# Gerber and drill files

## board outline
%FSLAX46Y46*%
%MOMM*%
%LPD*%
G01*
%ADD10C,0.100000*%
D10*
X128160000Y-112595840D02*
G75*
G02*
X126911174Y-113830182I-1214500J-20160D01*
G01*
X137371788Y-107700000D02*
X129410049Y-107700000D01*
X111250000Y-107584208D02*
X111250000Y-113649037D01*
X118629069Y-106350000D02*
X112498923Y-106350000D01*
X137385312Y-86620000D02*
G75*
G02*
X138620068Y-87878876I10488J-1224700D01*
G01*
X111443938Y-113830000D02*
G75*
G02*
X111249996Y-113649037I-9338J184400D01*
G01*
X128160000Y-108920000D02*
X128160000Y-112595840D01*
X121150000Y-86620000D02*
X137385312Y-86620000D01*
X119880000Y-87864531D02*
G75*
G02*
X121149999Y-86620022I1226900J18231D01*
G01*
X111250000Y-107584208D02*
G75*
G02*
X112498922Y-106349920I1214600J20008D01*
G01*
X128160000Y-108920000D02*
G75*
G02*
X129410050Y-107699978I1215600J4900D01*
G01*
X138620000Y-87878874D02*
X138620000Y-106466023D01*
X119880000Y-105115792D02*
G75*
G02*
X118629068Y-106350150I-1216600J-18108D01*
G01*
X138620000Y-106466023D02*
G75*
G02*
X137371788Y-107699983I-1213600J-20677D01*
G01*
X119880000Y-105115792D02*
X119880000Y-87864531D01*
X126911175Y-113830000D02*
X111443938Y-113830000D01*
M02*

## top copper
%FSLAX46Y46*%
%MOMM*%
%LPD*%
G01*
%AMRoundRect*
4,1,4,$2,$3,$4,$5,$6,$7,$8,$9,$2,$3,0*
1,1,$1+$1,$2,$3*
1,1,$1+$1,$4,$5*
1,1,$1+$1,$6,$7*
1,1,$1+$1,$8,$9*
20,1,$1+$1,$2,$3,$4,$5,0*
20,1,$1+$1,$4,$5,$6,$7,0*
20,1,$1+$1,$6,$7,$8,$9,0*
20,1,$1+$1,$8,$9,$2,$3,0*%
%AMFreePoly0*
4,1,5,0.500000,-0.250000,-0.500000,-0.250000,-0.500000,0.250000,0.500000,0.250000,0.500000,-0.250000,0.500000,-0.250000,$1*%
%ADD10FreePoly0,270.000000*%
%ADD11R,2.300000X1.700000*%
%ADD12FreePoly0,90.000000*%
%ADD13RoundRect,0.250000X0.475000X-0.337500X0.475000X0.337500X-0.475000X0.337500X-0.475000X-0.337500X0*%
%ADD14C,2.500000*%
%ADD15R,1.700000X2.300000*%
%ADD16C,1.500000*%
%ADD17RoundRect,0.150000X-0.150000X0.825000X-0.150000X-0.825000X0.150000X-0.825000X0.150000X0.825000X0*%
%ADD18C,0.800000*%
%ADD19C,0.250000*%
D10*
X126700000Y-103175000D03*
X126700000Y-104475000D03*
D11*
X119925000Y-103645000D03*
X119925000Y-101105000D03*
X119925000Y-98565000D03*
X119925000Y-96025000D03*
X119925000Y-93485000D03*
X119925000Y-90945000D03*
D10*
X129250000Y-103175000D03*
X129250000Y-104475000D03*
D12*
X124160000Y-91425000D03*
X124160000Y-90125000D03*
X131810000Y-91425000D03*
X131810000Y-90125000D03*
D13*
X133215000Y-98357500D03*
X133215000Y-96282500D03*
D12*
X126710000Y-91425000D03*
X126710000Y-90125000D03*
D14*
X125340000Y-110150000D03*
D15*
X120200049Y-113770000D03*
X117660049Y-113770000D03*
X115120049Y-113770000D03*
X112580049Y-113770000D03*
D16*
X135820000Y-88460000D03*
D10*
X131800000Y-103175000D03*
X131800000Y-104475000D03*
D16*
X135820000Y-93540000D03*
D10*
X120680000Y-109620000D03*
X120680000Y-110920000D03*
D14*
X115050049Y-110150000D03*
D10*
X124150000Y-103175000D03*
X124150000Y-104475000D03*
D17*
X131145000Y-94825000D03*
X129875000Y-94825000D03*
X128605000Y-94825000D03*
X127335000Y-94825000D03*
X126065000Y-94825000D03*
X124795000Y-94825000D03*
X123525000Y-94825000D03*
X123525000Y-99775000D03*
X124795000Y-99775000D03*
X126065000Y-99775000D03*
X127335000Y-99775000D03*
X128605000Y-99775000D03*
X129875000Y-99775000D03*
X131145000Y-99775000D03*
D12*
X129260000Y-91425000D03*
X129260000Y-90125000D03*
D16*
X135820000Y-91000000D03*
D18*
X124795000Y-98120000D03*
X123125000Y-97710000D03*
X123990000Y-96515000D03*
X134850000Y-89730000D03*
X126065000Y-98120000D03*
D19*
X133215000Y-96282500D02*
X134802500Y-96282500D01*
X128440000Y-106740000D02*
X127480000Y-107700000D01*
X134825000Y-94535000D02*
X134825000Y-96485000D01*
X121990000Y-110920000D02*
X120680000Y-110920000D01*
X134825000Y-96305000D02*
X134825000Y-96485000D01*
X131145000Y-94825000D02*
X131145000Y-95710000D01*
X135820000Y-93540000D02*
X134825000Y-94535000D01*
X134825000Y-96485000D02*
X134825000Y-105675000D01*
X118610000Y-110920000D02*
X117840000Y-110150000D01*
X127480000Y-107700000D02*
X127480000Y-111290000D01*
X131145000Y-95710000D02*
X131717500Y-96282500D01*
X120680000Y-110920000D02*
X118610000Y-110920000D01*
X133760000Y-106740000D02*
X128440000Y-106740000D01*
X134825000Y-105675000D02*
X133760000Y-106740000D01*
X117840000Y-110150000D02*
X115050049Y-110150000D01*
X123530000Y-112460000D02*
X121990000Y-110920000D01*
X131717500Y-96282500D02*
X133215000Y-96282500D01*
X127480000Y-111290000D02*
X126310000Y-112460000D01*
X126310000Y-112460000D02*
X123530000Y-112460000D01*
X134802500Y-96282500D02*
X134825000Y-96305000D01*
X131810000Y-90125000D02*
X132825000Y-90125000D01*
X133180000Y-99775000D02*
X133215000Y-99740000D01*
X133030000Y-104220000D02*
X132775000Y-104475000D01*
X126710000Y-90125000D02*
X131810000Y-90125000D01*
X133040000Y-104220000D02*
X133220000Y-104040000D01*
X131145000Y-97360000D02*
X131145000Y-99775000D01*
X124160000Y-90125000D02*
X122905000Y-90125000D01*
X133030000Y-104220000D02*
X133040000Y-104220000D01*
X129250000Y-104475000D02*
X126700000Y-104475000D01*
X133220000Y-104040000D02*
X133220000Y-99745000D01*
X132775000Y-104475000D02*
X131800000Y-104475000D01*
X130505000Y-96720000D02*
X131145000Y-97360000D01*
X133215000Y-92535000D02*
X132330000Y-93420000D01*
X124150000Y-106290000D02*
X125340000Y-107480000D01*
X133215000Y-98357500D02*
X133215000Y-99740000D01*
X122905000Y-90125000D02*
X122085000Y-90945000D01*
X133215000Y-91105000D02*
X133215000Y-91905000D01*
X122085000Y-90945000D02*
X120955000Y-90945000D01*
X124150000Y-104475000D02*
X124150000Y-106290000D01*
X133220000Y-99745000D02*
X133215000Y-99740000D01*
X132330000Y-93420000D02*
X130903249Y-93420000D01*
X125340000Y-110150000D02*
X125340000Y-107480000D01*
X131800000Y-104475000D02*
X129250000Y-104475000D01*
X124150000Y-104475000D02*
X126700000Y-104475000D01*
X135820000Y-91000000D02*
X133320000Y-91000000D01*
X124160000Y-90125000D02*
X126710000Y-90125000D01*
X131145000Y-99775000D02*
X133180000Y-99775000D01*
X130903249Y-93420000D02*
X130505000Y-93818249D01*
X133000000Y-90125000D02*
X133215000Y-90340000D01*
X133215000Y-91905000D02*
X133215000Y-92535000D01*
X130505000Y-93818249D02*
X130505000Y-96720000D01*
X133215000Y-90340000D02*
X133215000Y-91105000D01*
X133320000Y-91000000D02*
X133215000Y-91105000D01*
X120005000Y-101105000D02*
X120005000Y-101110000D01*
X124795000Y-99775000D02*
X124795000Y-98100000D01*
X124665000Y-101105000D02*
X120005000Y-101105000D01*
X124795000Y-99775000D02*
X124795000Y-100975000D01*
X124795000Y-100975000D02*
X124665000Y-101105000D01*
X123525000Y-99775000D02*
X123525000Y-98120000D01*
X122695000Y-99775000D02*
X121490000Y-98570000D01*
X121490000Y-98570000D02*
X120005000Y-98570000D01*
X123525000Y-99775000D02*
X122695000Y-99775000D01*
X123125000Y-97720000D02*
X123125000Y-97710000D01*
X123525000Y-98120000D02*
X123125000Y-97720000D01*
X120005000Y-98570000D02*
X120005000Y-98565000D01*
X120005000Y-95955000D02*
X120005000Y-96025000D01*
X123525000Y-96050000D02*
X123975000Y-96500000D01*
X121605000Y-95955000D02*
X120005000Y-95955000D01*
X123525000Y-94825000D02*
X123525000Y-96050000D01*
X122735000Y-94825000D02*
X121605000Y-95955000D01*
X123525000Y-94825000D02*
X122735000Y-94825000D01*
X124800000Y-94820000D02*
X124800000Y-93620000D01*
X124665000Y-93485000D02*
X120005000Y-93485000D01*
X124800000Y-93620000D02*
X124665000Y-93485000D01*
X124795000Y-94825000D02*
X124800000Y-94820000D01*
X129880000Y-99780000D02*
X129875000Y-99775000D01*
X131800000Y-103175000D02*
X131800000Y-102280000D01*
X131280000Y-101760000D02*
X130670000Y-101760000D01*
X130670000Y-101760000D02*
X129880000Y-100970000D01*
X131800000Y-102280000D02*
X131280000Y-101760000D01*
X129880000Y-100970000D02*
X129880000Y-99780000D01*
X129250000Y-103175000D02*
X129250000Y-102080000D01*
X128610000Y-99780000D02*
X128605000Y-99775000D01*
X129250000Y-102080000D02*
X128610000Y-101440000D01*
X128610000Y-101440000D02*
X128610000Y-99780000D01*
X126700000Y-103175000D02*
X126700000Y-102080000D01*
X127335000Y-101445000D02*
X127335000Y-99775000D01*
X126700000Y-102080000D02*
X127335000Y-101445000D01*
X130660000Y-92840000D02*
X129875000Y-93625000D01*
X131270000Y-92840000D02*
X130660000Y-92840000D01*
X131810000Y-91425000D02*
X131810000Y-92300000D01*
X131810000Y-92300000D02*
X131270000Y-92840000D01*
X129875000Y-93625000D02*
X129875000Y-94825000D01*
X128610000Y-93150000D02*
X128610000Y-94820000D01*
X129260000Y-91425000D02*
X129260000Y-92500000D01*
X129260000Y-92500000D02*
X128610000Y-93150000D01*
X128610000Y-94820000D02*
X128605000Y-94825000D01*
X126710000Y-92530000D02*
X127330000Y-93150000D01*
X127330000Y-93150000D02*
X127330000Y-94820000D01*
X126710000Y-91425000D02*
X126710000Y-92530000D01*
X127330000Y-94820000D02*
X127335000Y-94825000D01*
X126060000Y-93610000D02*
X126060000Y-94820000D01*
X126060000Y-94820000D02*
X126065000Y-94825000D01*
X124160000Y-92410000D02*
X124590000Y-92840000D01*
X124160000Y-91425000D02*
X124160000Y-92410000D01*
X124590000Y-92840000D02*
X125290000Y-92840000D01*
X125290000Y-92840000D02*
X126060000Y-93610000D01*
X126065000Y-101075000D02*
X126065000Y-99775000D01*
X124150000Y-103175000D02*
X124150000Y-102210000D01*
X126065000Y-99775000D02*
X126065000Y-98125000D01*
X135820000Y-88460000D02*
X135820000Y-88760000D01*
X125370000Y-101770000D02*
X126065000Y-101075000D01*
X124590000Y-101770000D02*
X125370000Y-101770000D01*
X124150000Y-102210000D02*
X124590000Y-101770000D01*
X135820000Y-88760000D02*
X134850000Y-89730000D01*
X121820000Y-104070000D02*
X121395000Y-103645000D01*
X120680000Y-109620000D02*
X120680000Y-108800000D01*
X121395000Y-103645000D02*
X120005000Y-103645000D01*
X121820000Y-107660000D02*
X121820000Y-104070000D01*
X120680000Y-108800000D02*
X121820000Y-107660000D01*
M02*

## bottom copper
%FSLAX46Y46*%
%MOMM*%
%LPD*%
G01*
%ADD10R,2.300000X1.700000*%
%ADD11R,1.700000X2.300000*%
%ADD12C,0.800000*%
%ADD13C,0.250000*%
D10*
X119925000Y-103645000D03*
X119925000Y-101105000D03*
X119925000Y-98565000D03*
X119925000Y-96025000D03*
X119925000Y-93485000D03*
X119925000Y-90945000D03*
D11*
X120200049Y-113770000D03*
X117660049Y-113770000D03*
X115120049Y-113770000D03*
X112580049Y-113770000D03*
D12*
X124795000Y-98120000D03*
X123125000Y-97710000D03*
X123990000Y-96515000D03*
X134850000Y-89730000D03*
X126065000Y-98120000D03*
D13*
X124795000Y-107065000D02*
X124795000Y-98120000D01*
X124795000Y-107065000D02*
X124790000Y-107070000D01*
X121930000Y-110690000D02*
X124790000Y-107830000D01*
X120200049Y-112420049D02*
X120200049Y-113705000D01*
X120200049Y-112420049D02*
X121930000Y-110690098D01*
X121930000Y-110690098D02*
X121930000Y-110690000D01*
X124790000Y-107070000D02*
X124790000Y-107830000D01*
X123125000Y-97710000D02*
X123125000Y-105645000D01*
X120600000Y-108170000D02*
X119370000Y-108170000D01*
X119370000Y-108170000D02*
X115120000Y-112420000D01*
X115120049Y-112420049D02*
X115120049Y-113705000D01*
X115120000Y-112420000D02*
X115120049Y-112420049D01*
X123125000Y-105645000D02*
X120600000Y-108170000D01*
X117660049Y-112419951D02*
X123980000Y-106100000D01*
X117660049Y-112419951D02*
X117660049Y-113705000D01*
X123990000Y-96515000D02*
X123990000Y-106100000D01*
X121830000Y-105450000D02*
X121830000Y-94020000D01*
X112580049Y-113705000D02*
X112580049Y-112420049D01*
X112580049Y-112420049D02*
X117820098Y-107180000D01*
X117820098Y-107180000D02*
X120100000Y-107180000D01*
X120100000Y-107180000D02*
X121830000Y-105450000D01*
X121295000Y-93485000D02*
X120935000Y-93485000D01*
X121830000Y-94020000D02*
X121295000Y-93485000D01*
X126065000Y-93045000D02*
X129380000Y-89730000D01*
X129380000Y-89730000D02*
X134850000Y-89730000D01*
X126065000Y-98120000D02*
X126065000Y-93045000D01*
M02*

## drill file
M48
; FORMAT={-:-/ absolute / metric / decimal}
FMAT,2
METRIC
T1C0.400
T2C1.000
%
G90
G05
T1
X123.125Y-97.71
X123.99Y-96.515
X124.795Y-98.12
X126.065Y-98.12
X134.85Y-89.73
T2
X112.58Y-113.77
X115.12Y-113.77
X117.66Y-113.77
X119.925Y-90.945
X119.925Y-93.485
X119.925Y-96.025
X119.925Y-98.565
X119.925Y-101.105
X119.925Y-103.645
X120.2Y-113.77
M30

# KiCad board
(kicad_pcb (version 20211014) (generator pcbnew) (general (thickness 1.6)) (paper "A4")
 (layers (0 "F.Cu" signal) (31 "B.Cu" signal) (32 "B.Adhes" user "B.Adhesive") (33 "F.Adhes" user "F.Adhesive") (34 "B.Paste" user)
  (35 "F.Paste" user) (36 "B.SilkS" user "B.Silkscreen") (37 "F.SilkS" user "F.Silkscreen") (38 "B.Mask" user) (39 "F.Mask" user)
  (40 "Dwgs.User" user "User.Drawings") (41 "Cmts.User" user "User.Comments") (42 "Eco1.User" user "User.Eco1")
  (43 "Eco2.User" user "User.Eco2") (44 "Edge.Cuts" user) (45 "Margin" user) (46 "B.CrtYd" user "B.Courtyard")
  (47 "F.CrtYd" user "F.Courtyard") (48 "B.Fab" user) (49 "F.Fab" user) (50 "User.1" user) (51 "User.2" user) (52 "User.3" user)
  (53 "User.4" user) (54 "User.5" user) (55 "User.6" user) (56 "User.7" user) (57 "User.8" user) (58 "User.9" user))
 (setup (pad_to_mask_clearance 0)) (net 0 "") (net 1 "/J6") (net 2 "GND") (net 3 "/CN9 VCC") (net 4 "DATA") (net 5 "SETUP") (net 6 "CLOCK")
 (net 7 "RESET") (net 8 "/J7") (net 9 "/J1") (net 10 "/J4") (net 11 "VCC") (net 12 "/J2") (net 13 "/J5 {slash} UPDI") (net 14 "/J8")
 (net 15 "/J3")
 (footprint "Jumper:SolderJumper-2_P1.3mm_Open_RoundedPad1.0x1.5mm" (layer "F.Cu") (at 126.7 103.825 -90)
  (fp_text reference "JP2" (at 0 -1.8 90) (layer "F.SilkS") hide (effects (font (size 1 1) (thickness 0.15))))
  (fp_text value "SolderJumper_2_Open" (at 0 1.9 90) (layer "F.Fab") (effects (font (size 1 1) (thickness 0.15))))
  (pad "1" smd custom (at -0.65 0 270) (size 1 0.5) (layers "F.Cu" "F.Mask") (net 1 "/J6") (zone_connect 2)
   (options (clearance outline) (anchor rect)) (primitives))
  (pad "2" smd custom (at 0.65 0 270) (size 1 0.5) (layers "F.Cu" "F.Mask") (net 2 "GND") (zone_connect 2)
   (options (clearance outline) (anchor rect)) (primitives)))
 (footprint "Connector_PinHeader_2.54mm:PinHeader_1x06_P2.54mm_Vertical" (layer "F.Cu") (at 119.925 103.645 180)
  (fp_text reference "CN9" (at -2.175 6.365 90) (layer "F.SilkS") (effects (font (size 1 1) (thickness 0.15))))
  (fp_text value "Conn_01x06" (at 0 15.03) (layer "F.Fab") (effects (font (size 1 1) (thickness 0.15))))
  (pad "1" thru_hole rect (at 0 0 180) (size 2.3 1.7) (drill 1) (layers *.Cu *.Mask) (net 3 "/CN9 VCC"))
  (pad "2" thru_hole rect (at 0 2.54 180) (size 2.3 1.7) (drill 1) (layers *.Cu *.Mask) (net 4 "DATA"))
  (pad "3" thru_hole rect (at 0 5.08 180) (size 2.3 1.7) (drill 1) (layers *.Cu *.Mask) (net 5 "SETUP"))
  (pad "4" thru_hole rect (at 0 7.62 180) (size 2.3 1.7) (drill 1) (layers *.Cu *.Mask) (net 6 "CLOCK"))
  (pad "5" thru_hole rect (at 0 10.16 180) (size 2.3 1.7) (drill 1) (layers *.Cu *.Mask) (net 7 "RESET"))
  (pad "6" thru_hole rect (at 0 12.7 180) (size 2.3 1.7) (drill 1) (layers *.Cu *.Mask) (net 2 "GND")))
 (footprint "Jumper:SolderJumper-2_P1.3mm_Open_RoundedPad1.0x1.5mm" (layer "F.Cu") (at 129.25 103.825 -90)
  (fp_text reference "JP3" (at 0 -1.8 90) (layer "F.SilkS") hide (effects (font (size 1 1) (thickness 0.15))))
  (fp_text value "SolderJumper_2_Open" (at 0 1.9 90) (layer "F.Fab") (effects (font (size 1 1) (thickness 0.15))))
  (pad "1" smd custom (at -0.65 0 270) (size 1 0.5) (layers "F.Cu" "F.Mask") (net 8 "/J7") (zone_connect 2)
   (options (clearance outline) (anchor rect)) (primitives))
  (pad "2" smd custom (at 0.65 0 270) (size 1 0.5) (layers "F.Cu" "F.Mask") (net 2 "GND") (zone_connect 2)
   (options (clearance outline) (anchor rect)) (primitives)))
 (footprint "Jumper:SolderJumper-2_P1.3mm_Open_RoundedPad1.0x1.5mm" (layer "F.Cu") (at 124.16 90.775 90)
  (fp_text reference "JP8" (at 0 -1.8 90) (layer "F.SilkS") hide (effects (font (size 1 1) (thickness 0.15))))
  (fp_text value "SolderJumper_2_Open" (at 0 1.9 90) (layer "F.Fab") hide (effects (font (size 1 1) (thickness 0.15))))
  (pad "1" smd custom (at -0.65 0 90) (size 1 0.5) (layers "F.Cu" "F.Mask") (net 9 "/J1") (zone_connect 2)
   (options (clearance outline) (anchor rect)) (primitives))
  (pad "2" smd custom (at 0.65 0 90) (size 1 0.5) (layers "F.Cu" "F.Mask") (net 2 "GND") (zone_connect 2)
   (options (clearance outline) (anchor rect)) (primitives)))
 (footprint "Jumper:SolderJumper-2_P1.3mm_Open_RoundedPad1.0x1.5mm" (layer "F.Cu") (at 131.81 90.775 90)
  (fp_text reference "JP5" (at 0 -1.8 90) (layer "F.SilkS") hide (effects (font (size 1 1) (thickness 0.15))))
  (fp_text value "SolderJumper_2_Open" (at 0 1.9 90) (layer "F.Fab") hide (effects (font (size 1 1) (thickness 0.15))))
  (pad "1" smd custom (at -0.65 0 90) (size 1 0.5) (layers "F.Cu" "F.Mask") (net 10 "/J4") (zone_connect 2)
   (options (clearance outline) (anchor rect)) (primitives))
  (pad "2" smd custom (at 0.65 0 90) (size 1 0.5) (layers "F.Cu" "F.Mask") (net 2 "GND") (zone_connect 2)
   (options (clearance outline) (anchor rect)) (primitives)))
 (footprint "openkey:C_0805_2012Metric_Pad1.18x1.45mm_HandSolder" (layer "F.Cu") (at 133.215 97.32 90)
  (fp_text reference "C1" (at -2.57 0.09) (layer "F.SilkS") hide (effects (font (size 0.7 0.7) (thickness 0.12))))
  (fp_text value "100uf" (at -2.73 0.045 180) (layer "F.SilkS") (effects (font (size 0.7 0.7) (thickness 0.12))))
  (pad "1" smd roundrect (at -1.0375 0 90) (size 1.175 1.45) (layers "F.Cu" "F.Paste" "F.Mask") (roundrect_rratio 0.2127659574)
   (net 2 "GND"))
  (pad "2" smd roundrect (at 1.0375 0 90) (size 1.175 1.45) (layers "F.Cu" "F.Paste" "F.Mask") (roundrect_rratio 0.2127659574)
   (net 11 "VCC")))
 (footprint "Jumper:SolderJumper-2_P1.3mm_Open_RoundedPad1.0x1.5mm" (layer "F.Cu") (at 126.71 90.775 90)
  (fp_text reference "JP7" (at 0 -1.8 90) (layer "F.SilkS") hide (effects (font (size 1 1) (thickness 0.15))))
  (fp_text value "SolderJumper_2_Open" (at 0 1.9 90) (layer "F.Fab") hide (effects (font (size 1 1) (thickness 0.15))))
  (pad "1" smd custom (at -0.65 0 90) (size 1 0.5) (layers "F.Cu" "F.Mask") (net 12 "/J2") (zone_connect 2)
   (options (clearance outline) (anchor rect)) (primitives))
  (pad "2" smd custom (at 0.65 0 90) (size 1 0.5) (layers "F.Cu" "F.Mask") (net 2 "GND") (zone_connect 2)
   (options (clearance outline) (anchor rect)) (primitives)))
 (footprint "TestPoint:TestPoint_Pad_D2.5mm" (layer "F.Cu") (at 125.34 110.12)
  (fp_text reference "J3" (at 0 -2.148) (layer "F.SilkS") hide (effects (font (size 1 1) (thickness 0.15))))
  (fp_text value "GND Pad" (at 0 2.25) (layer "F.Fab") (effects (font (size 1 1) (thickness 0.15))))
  (pad "1" smd circle (at 0 0.03) (size 2.5 2.5) (layers "F.Cu" "F.Mask") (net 2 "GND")))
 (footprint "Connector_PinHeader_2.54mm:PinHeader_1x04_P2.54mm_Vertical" (layer "F.Cu") (at 120.200049 113.77 -90)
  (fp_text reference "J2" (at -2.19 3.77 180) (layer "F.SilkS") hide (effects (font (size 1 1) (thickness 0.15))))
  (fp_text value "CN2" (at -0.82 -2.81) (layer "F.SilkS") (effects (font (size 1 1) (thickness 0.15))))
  (pad "1" thru_hole rect (at 0 0 270) (size 2.3 1.7) (drill 1) (layers *.Cu *.Mask) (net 4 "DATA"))
  (pad "2" thru_hole rect (at 0 2.54 270) (size 2.3 1.7) (drill 1) (layers *.Cu *.Mask) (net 6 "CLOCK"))
  (pad "3" thru_hole rect (at 0 5.08 270) (size 2.3 1.7) (drill 1) (layers *.Cu *.Mask) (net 5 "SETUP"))
  (pad "4" thru_hole rect (at 0 7.62 270) (size 2.3 1.7) (drill 1) (layers *.Cu *.Mask) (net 7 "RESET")))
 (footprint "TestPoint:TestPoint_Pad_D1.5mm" (layer "F.Cu") (at 135.82 88.46 90)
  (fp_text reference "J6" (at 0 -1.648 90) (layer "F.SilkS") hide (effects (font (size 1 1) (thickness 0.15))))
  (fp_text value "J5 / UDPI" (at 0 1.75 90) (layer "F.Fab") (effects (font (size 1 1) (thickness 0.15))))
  (pad "1" smd circle (at 0 0 90) (size 1.5 1.5) (layers "F.Cu" "F.Mask") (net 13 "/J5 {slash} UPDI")))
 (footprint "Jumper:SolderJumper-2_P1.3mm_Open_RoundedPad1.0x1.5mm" (layer "F.Cu") (at 131.8 103.825 -90)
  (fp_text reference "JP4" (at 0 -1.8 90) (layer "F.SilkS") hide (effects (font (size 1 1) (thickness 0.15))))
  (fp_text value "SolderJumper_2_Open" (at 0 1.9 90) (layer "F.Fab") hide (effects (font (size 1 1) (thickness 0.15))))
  (pad "1" smd custom (at -0.65 0 270) (size 1 0.5) (layers "F.Cu" "F.Mask") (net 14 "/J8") (zone_connect 2)
   (options (clearance outline) (anchor rect)) (primitives))
  (pad "2" smd custom (at 0.65 0 270) (size 1 0.5) (layers "F.Cu" "F.Mask") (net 2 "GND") (zone_connect 2)
   (options (clearance outline) (anchor rect)) (primitives)))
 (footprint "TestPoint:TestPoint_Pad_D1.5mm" (layer "F.Cu") (at 135.82 93.54 90)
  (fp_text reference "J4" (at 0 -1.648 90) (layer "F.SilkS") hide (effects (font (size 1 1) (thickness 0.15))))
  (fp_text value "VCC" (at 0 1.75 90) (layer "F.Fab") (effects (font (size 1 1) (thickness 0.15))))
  (pad "1" smd circle (at 0 0 90) (size 1.5 1.5) (layers "F.Cu" "F.Mask") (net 11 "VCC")))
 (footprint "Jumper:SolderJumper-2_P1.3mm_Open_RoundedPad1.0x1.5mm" (layer "F.Cu") (at 120.68 110.27 -90)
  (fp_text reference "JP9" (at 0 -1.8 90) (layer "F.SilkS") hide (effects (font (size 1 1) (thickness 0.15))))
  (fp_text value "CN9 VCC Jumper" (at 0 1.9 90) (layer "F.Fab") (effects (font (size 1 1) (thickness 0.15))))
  (pad "1" smd custom (at -0.65 0 270) (size 1 0.5) (layers "F.Cu" "F.Mask") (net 3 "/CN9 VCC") (zone_connect 2)
   (options (clearance outline) (anchor rect)) (primitives))
  (pad "2" smd custom (at 0.65 0 270) (size 1 0.5) (layers "F.Cu" "F.Mask") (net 11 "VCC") (zone_connect 2)
   (options (clearance outline) (anchor rect)) (primitives)))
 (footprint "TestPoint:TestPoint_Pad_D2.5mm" (layer "F.Cu") (at 115.050049 110.15 90)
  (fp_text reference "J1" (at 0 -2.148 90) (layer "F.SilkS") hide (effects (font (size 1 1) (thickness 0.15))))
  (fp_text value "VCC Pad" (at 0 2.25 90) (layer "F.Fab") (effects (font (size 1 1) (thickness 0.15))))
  (pad "1" smd circle (at 0 0 90) (size 2.5 2.5) (layers "F.Cu" "F.Mask") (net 11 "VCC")))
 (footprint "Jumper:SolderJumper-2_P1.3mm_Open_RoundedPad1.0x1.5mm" (layer "F.Cu") (at 124.15 103.825 -90)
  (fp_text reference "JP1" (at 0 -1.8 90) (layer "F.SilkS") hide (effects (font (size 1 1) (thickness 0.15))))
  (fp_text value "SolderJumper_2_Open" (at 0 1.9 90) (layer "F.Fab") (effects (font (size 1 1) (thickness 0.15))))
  (pad "1" smd custom (at -0.65 0 270) (size 1 0.5) (layers "F.Cu" "F.Mask") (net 13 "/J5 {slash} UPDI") (zone_connect 2)
   (options (clearance outline) (anchor rect)) (primitives))
  (pad "2" smd custom (at 0.65 0 270) (size 1 0.5) (layers "F.Cu" "F.Mask") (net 2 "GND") (zone_connect 2)
   (options (clearance outline) (anchor rect)) (primitives)))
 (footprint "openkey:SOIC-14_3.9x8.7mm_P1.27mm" (layer "F.Cu") (at 127.335 97.3 -90)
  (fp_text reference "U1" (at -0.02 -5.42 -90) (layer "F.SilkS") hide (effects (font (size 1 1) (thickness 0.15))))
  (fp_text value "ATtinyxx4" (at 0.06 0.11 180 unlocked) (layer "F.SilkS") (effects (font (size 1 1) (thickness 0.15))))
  (pad "1" smd roundrect (at -2.475 -3.81 270) (size 1.95 0.6) (layers "F.Cu" "F.Paste" "F.Mask") (roundrect_rratio 0.25) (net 11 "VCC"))
  (pad "2" smd roundrect (at -2.475 -2.54 270) (size 1.95 0.6) (layers "F.Cu" "F.Paste" "F.Mask") (roundrect_rratio 0.25) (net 10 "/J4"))
  (pad "3" smd roundrect (at -2.475 -1.27 270) (size 1.95 0.6) (layers "F.Cu" "F.Paste" "F.Mask") (roundrect_rratio 0.25) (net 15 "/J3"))
  (pad "4" smd roundrect (at -2.475 0 270) (size 1.95 0.6) (layers "F.Cu" "F.Paste" "F.Mask") (roundrect_rratio 0.25) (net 12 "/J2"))
  (pad "5" smd roundrect (at -2.475 1.27 270) (size 1.95 0.6) (layers "F.Cu" "F.Paste" "F.Mask") (roundrect_rratio 0.25) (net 9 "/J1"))
  (pad "6" smd roundrect (at -2.475 2.54 270) (size 1.95 0.6) (layers "F.Cu" "F.Paste" "F.Mask") (roundrect_rratio 0.25) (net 7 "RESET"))
  (pad "7" smd roundrect (at -2.475 3.81 270) (size 1.95 0.6) (layers "F.Cu" "F.Paste" "F.Mask") (roundrect_rratio 0.25) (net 6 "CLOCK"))
  (pad "8" smd roundrect (at 2.475 3.81 270) (size 1.95 0.6) (layers "F.Cu" "F.Paste" "F.Mask") (roundrect_rratio 0.25) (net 5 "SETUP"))
  (pad "9" smd roundrect (at 2.475 2.54 270) (size 1.95 0.6) (layers "F.Cu" "F.Paste" "F.Mask") (roundrect_rratio 0.25) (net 4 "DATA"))
  (pad "10" smd roundrect (at 2.475 1.27 270) (size 1.95 0.6) (layers "F.Cu" "F.Paste" "F.Mask") (roundrect_rratio 0.25)
   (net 13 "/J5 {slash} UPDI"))
  (pad "11" smd roundrect (at 2.475 0 270) (size 1.95 0.6) (layers "F.Cu" "F.Paste" "F.Mask") (roundrect_rratio 0.25) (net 1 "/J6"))
  (pad "12" smd roundrect (at 2.475 -1.27 270) (size 1.95 0.6) (layers "F.Cu" "F.Paste" "F.Mask") (roundrect_rratio 0.25) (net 8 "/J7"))
  (pad "13" smd roundrect (at 2.475 -2.54 270) (size 1.95 0.6) (layers "F.Cu" "F.Paste" "F.Mask") (roundrect_rratio 0.25) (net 14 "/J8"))
  (pad "14" smd roundrect (at 2.475 -3.81 270) (size 1.95 0.6) (layers "F.Cu" "F.Paste" "F.Mask") (roundrect_rratio 0.25) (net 2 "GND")))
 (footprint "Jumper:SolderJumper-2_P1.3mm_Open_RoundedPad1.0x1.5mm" (layer "F.Cu") (at 129.26 90.775 90)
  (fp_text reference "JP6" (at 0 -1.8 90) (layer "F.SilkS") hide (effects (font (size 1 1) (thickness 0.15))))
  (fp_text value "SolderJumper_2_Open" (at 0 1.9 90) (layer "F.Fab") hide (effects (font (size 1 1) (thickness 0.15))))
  (pad "1" smd custom (at -0.65 0 90) (size 1 0.5) (layers "F.Cu" "F.Mask") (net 15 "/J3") (zone_connect 2)
   (options (clearance outline) (anchor rect)) (primitives))
  (pad "2" smd custom (at 0.65 0 90) (size 1 0.5) (layers "F.Cu" "F.Mask") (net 2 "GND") (zone_connect 2)
   (options (clearance outline) (anchor rect)) (primitives)))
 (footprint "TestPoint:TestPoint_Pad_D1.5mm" (layer "F.Cu") (at 135.82 91 90)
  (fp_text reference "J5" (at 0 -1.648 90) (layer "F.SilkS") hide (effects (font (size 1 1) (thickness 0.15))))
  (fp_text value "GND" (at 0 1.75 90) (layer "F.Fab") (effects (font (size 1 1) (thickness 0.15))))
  (pad "1" smd circle (at 0 0 90) (size 1.5 1.5) (layers "F.Cu" "F.Mask") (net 2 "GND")))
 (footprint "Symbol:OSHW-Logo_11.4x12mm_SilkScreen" (layer "B.Cu") (at 129.87 98.2 180)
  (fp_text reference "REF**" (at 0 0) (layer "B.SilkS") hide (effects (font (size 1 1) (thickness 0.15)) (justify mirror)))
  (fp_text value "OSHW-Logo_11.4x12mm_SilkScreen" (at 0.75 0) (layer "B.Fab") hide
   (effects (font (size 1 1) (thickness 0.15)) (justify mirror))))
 (gr_arc (start 128.16 112.59584) (mid 127.799359 113.479869) (end 126.911175 113.830151) (layer "Edge.Cuts") (width 0.1))
 (gr_line (start 137.371788 107.7) (end 129.410049 107.7) (layer "Edge.Cuts") (width 0.1))
 (gr_line (start 111.25 107.584208) (end 111.25 113.649037) (layer "Edge.Cuts") (width 0.1))
 (gr_line (start 118.629069 106.35) (end 112.498923 106.35) (layer "Edge.Cuts") (width 0.1))
 (gr_arc (start 137.385312 86.62) (mid 138.270129 86.987103) (end 138.62 87.878874) (layer "Edge.Cuts") (width 0.1))
 (gr_arc (start 111.443938 113.83) (mid 111.308653 113.780581) (end 111.25 113.649037) (layer "Edge.Cuts") (width 0.1))
 (gr_line (start 128.16 108.92) (end 128.16 112.59584) (layer "Edge.Cuts") (width 0.1))
 (gr_line (start 121.15 86.62) (end 137.385312 86.62) (layer "Edge.Cuts") (width 0.1))
 (gr_arc (start 119.88 87.864531) (mid 120.248097 86.969901) (end 121.15 86.62) (layer "Edge.Cuts") (width 0.1))
 (gr_arc (start 111.25 107.584208) (mid 111.610701 106.70017) (end 112.498923 106.349897) (layer "Edge.Cuts") (width 0.1))
 (gr_arc (start 128.16 108.92) (mid 128.526543 108.045152) (end 129.410049 107.7) (layer "Edge.Cuts") (width 0.1))
 (gr_line (start 138.62 87.878874) (end 138.62 106.466023) (layer "Edge.Cuts") (width 0.1))
 (gr_arc (start 119.88 105.115792) (mid 119.518002 105.999964) (end 118.629069 106.350103) (layer "Edge.Cuts") (width 0.1))
 (gr_arc (start 138.62 106.466023) (mid 138.259719 107.34988) (end 137.371788 107.7) (layer "Edge.Cuts") (width 0.1))
 (gr_line (start 119.88 105.115792) (end 119.88 87.864531) (layer "Edge.Cuts") (width 0.1))
 (gr_line (start 126.911175 113.83) (end 111.443938 113.83) (layer "Edge.Cuts") (width 0.1))
 (segment (start 133.215 96.2825) (end 134.8025 96.2825) (width 0.25) (layer "F.Cu") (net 11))
 (segment (start 128.44 106.74) (end 127.48 107.7) (width 0.25) (layer "F.Cu") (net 11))
 (segment (start 134.825 94.535) (end 134.825 96.485) (width 0.25) (layer "F.Cu") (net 11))
 (segment (start 121.99 110.92) (end 120.68 110.92) (width 0.25) (layer "F.Cu") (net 11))
 (segment (start 134.825 96.305) (end 134.825 96.485) (width 0.25) (layer "F.Cu") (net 11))
 (segment (start 131.145 94.825) (end 131.145 95.71) (width 0.25) (layer "F.Cu") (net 11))
 (segment (start 135.82 93.54) (end 134.825 94.535) (width 0.25) (layer "F.Cu") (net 11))
 (segment (start 134.825 96.485) (end 134.825 105.675) (width 0.25) (layer "F.Cu") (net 11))
 (segment (start 118.61 110.92) (end 117.84 110.15) (width 0.25) (layer "F.Cu") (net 11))
 (segment (start 127.48 107.7) (end 127.48 111.29) (width 0.25) (layer "F.Cu") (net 11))
 (segment (start 131.145 95.71) (end 131.7175 96.2825) (width 0.25) (layer "F.Cu") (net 11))
 (segment (start 120.68 110.92) (end 118.61 110.92) (width 0.25) (layer "F.Cu") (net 11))
 (segment (start 133.76 106.74) (end 128.44 106.74) (width 0.25) (layer "F.Cu") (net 11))
 (segment (start 134.825 105.675) (end 133.76 106.74) (width 0.25) (layer "F.Cu") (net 11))
 (segment (start 117.84 110.15) (end 115.050049 110.15) (width 0.25) (layer "F.Cu") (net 11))
 (segment (start 123.53 112.46) (end 121.99 110.92) (width 0.25) (layer "F.Cu") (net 11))
 (segment (start 131.7175 96.2825) (end 133.215 96.2825) (width 0.25) (layer "F.Cu") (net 11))
 (segment (start 127.48 111.29) (end 126.31 112.46) (width 0.25) (layer "F.Cu") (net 11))
 (segment (start 126.31 112.46) (end 123.53 112.46) (width 0.25) (layer "F.Cu") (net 11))
 (segment (start 134.8025 96.2825) (end 134.825 96.305) (width 0.25) (layer "F.Cu") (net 11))
 (segment (start 131.81 90.125) (end 132.825 90.125) (width 0.25) (layer "F.Cu") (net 2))
 (segment (start 133.18 99.775) (end 133.215 99.74) (width 0.25) (layer "F.Cu") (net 2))
 (segment (start 133.03 104.22) (end 132.775 104.475) (width 0.25) (layer "F.Cu") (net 2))
 (segment (start 126.71 90.125) (end 131.81 90.125) (width 0.25) (layer "F.Cu") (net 2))
 (segment (start 133.04 104.22) (end 133.22 104.04) (width 0.25) (layer "F.Cu") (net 2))
 (segment (start 131.145 97.36) (end 131.145 99.775) (width 0.25) (layer "F.Cu") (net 2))
 (segment (start 124.16 90.125) (end 122.905 90.125) (width 0.25) (layer "F.Cu") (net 2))
 (segment (start 133.03 104.22) (end 133.04 104.22) (width 0.25) (layer "F.Cu") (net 2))
 (segment (start 129.25 104.475) (end 126.7 104.475) (width 0.25) (layer "F.Cu") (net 2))
 (segment (start 133.22 104.04) (end 133.22 99.745) (width 0.25) (layer "F.Cu") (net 2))
 (segment (start 132.775 104.475) (end 131.8 104.475) (width 0.25) (layer "F.Cu") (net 2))
 (segment (start 130.505 96.72) (end 131.145 97.36) (width 0.25) (layer "F.Cu") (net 2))
 (segment (start 133.215 92.535) (end 132.33 93.42) (width 0.25) (layer "F.Cu") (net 2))
 (segment (start 124.15 106.29) (end 125.34 107.48) (width 0.25) (layer "F.Cu") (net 2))
 (segment (start 133.215 98.3575) (end 133.215 99.74) (width 0.25) (layer "F.Cu") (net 2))
 (segment (start 122.905 90.125) (end 122.085 90.945) (width 0.25) (layer "F.Cu") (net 2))
 (segment (start 133.215 91.105) (end 133.215 91.905) (width 0.25) (layer "F.Cu") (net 2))
 (segment (start 122.085 90.945) (end 120.955 90.945) (width 0.25) (layer "F.Cu") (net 2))
 (segment (start 124.15 104.475) (end 124.15 106.29) (width 0.25) (layer "F.Cu") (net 2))
 (segment (start 133.22 99.745) (end 133.215 99.74) (width 0.25) (layer "F.Cu") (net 2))
 (segment (start 132.33 93.42) (end 130.903249 93.42) (width 0.25) (layer "F.Cu") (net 2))
 (segment (start 125.34 110.15) (end 125.34 107.48) (width 0.25) (layer "F.Cu") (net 2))
 (segment (start 131.8 104.475) (end 129.25 104.475) (width 0.25) (layer "F.Cu") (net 2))
 (segment (start 124.15 104.475) (end 126.7 104.475) (width 0.25) (layer "F.Cu") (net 2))
 (segment (start 135.82 91) (end 133.32 91) (width 0.25) (layer "F.Cu") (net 2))
 (segment (start 124.16 90.125) (end 126.71 90.125) (width 0.25) (layer "F.Cu") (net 2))
 (segment (start 131.145 99.775) (end 133.18 99.775) (width 0.25) (layer "F.Cu") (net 2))
 (segment (start 130.903249 93.42) (end 130.505 93.818249) (width 0.25) (layer "F.Cu") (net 2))
 (segment (start 133 90.125) (end 133.215 90.34) (width 0.25) (layer "F.Cu") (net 2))
 (segment (start 133.215 91.905) (end 133.215 92.535) (width 0.25) (layer "F.Cu") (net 2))
 (segment (start 130.505 93.818249) (end 130.505 96.72) (width 0.25) (layer "F.Cu") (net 2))
 (segment (start 133.215 90.34) (end 133.215 91.105) (width 0.25) (layer "F.Cu") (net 2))
 (segment (start 133.32 91) (end 133.215 91.105) (width 0.25) (layer "F.Cu") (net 2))
 (segment (start 120.005 101.105) (end 120.005 101.11) (width 0.25) (layer "F.Cu") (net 4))
 (segment (start 124.795 99.775) (end 124.795 98.1) (width 0.25) (layer "F.Cu") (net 4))
 (segment (start 124.665 101.105) (end 120.005 101.105) (width 0.25) (layer "F.Cu") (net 4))
 (segment (start 124.795 99.775) (end 124.795 100.975) (width 0.25) (layer "F.Cu") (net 4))
 (segment (start 124.795 100.975) (end 124.665 101.105) (width 0.25) (layer "F.Cu") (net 4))
 (via (at 124.795 98.12) (size 0.8) (drill 0.4) (layers "F.Cu" "B.Cu") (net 4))
 (segment (start 124.795 107.065) (end 124.795 98.12) (width 0.25) (layer "B.Cu") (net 4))
 (segment (start 124.795 107.065) (end 124.79 107.07) (width 0.25) (layer "B.Cu") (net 4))
 (segment (start 121.93 110.69) (end 124.79 107.83) (width 0.25) (layer "B.Cu") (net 4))
 (segment (start 120.200049 112.420049) (end 120.200049 113.705) (width 0.25) (layer "B.Cu") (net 4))
 (segment (start 120.200049 112.420049) (end 121.93 110.690098) (width 0.25) (layer "B.Cu") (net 4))
 (segment (start 121.93 110.690098) (end 121.93 110.69) (width 0.25) (layer "B.Cu") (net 4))
 (segment (start 124.79 107.07) (end 124.79 107.83) (width 0.25) (layer "B.Cu") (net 4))
 (segment (start 123.525 99.775) (end 123.525 98.12) (width 0.25) (layer "F.Cu") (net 5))
 (segment (start 122.695 99.775) (end 121.49 98.57) (width 0.25) (layer "F.Cu") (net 5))
 (segment (start 121.49 98.57) (end 120.005 98.57) (width 0.25) (layer "F.Cu") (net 5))
 (segment (start 123.525 99.775) (end 122.695 99.775) (width 0.25) (layer "F.Cu") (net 5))
 (segment (start 123.125 97.72) (end 123.125 97.71) (width 0.25) (layer "F.Cu") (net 5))
 (segment (start 123.525 98.12) (end 123.125 97.72) (width 0.25) (layer "F.Cu") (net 5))
 (segment (start 120.005 98.57) (end 120.005 98.565) (width 0.25) (layer "F.Cu") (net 5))
 (via (at 123.125 97.71) (size 0.8) (drill 0.4) (layers "F.Cu" "B.Cu") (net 5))
 (segment (start 123.125 97.71) (end 123.125 105.645) (width 0.25) (layer "B.Cu") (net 5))
 (segment (start 120.6 108.17) (end 119.37 108.17) (width 0.25) (layer "B.Cu") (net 5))
 (segment (start 119.37 108.17) (end 115.12 112.42) (width 0.25) (layer "B.Cu") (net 5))
 (segment (start 115.120049 112.420049) (end 115.120049 113.705) (width 0.25) (layer "B.Cu") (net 5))
 (segment (start 115.12 112.42) (end 115.120049 112.420049) (width 0.25) (layer "B.Cu") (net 5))
 (segment (start 123.125 105.645) (end 120.6 108.17) (width 0.25) (layer "B.Cu") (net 5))
 (segment (start 120.005 95.955) (end 120.005 96.025) (width 0.25) (layer "F.Cu") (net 6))
 (segment (start 123.525 96.05) (end 123.975 96.5) (width 0.25) (layer "F.Cu") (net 6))
 (segment (start 121.605 95.955) (end 120.005 95.955) (width 0.25) (layer "F.Cu") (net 6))
 (segment (start 123.525 94.825) (end 123.525 96.05) (width 0.25) (layer "F.Cu") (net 6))
 (segment (start 122.735 94.825) (end 121.605 95.955) (width 0.25) (layer "F.Cu") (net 6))
 (segment (start 123.525 94.825) (end 122.735 94.825) (width 0.25) (layer "F.Cu") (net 6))
 (via (at 123.99 96.515) (size 0.8) (drill 0.4) (layers "F.Cu" "B.Cu") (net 6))
 (segment (start 117.660049 112.419951) (end 123.98 106.1) (width 0.25) (layer "B.Cu") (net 6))
 (segment (start 117.660049 112.419951) (end 117.660049 113.705) (width 0.25) (layer "B.Cu") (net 6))
 (segment (start 123.99 96.515) (end 123.99 106.1) (width 0.25) (layer "B.Cu") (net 6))
 (segment (start 124.8 94.82) (end 124.8 93.62) (width 0.25) (layer "F.Cu") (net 7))
 (segment (start 124.665 93.485) (end 120.005 93.485) (width 0.25) (layer "F.Cu") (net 7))
 (segment (start 124.8 93.62) (end 124.665 93.485) (width 0.25) (layer "F.Cu") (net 7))
 (segment (start 124.795 94.825) (end 124.8 94.82) (width 0.25) (layer "F.Cu") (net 7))
 (segment (start 121.83 105.45) (end 121.83 94.02) (width 0.25) (layer "B.Cu") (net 7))
 (segment (start 112.580049 113.705) (end 112.580049 112.420049) (width 0.25) (layer "B.Cu") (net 7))
 (segment (start 112.580049 112.420049) (end 117.820098 107.18) (width 0.25) (layer "B.Cu") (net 7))
 (segment (start 117.820098 107.18) (end 120.1 107.18) (width 0.25) (layer "B.Cu") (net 7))
 (segment (start 120.1 107.18) (end 121.83 105.45) (width 0.25) (layer "B.Cu") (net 7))
 (segment (start 121.295 93.485) (end 120.935 93.485) (width 0.25) (layer "B.Cu") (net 7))
 (segment (start 121.83 94.02) (end 121.295 93.485) (width 0.25) (layer "B.Cu") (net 7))
 (segment (start 129.88 99.78) (end 129.875 99.775) (width 0.25) (layer "F.Cu") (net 14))
 (segment (start 131.8 103.175) (end 131.8 102.28) (width 0.25) (layer "F.Cu") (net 14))
 (segment (start 131.28 101.76) (end 130.67 101.76) (width 0.25) (layer "F.Cu") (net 14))
 (segment (start 130.67 101.76) (end 129.88 100.97) (width 0.25) (layer "F.Cu") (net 14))
 (segment (start 131.8 102.28) (end 131.28 101.76) (width 0.25) (layer "F.Cu") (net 14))
 (segment (start 129.88 100.97) (end 129.88 99.78) (width 0.25) (layer "F.Cu") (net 14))
 (segment (start 129.25 103.175) (end 129.25 102.08) (width 0.25) (layer "F.Cu") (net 8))
 (segment (start 128.61 99.78) (end 128.605 99.775) (width 0.25) (layer "F.Cu") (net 8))
 (segment (start 129.25 102.08) (end 128.61 101.44) (width 0.25) (layer "F.Cu") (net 8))
 (segment (start 128.61 101.44) (end 128.61 99.78) (width 0.25) (layer "F.Cu") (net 8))
 (segment (start 126.7 103.175) (end 126.7 102.08) (width 0.25) (layer "F.Cu") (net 1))
 (segment (start 127.335 101.445) (end 127.335 99.775) (width 0.25) (layer "F.Cu") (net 1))
 (segment (start 126.7 102.08) (end 127.335 101.445) (width 0.25) (layer "F.Cu") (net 1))
 (segment (start 130.66 92.84) (end 129.875 93.625) (width 0.25) (layer "F.Cu") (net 10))
 (segment (start 131.27 92.84) (end 130.66 92.84) (width 0.25) (layer "F.Cu") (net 10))
 (segment (start 131.81 91.425) (end 131.81 92.3) (width 0.25) (layer "F.Cu") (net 10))
 (segment (start 131.81 92.3) (end 131.27 92.84) (width 0.25) (layer "F.Cu") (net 10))
 (segment (start 129.875 93.625) (end 129.875 94.825) (width 0.25) (layer "F.Cu") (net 10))
 (segment (start 128.61 93.15) (end 128.61 94.82) (width 0.25) (layer "F.Cu") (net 15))
 (segment (start 129.26 91.425) (end 129.26 92.5) (width 0.25) (layer "F.Cu") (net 15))
 (segment (start 129.26 92.5) (end 128.61 93.15) (width 0.25) (layer "F.Cu") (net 15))
 (segment (start 128.61 94.82) (end 128.605 94.825) (width 0.25) (layer "F.Cu") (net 15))
 (segment (start 126.71 92.53) (end 127.33 93.15) (width 0.25) (layer "F.Cu") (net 12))
 (segment (start 127.33 93.15) (end 127.33 94.82) (width 0.25) (layer "F.Cu") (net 12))
 (segment (start 126.71 91.425) (end 126.71 92.53) (width 0.25) (layer "F.Cu") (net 12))
 (segment (start 127.33 94.82) (end 127.335 94.825) (width 0.25) (layer "F.Cu") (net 12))
 (segment (start 126.06 93.61) (end 126.06 94.82) (width 0.25) (layer "F.Cu") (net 9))
 (segment (start 126.06 94.82) (end 126.065 94.825) (width 0.25) (layer "F.Cu") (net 9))
 (segment (start 124.16 92.41) (end 124.59 92.84) (width 0.25) (layer "F.Cu") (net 9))
 (segment (start 124.16 91.425) (end 124.16 92.41) (width 0.25) (layer "F.Cu") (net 9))
 (segment (start 124.59 92.84) (end 125.29 92.84) (width 0.25) (layer "F.Cu") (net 9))
 (segment (start 125.29 92.84) (end 126.06 93.61) (width 0.25) (layer "F.Cu") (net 9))
 (segment (start 126.065 101.075) (end 126.065 99.775) (width 0.25) (layer "F.Cu") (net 13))
 (segment (start 124.15 103.175) (end 124.15 102.21) (width 0.25) (layer "F.Cu") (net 13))
 (segment (start 126.065 99.775) (end 126.065 98.125) (width 0.25) (layer "F.Cu") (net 13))
 (segment (start 135.82 88.46) (end 135.82 88.76) (width 0.25) (layer "F.Cu") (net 13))
 (segment (start 125.37 101.77) (end 126.065 101.075) (width 0.25) (layer "F.Cu") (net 13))
 (segment (start 124.59 101.77) (end 125.37 101.77) (width 0.25) (layer "F.Cu") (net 13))
 (segment (start 124.15 102.21) (end 124.59 101.77) (width 0.25) (layer "F.Cu") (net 13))
 (segment (start 135.82 88.76) (end 134.85 89.73) (width 0.25) (layer "F.Cu") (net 13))
 (via (at 134.85 89.73) (size 0.8) (drill 0.4) (layers "F.Cu" "B.Cu") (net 13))
 (via (at 126.065 98.12) (size 0.8) (drill 0.4) (layers "F.Cu" "B.Cu") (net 13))
 (segment (start 126.065 93.045) (end 129.38 89.73) (width 0.25) (layer "B.Cu") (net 13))
 (segment (start 129.38 89.73) (end 134.85 89.73) (width 0.25) (layer "B.Cu") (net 13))
 (segment (start 126.065 98.12) (end 126.065 93.045) (width 0.25) (layer "B.Cu") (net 13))
 (segment (start 121.82 104.07) (end 121.395 103.645) (width 0.25) (layer "F.Cu") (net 3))
 (segment (start 120.68 109.62) (end 120.68 108.8) (width 0.25) (layer "F.Cu") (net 3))
 (segment (start 121.395 103.645) (end 120.005 103.645) (width 0.25) (layer "F.Cu") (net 3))
 (segment (start 121.82 107.66) (end 121.82 104.07) (width 0.25) (layer "F.Cu") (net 3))
 (segment (start 120.68 108.8) (end 121.82 107.66) (width 0.25) (layer "F.Cu") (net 3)))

